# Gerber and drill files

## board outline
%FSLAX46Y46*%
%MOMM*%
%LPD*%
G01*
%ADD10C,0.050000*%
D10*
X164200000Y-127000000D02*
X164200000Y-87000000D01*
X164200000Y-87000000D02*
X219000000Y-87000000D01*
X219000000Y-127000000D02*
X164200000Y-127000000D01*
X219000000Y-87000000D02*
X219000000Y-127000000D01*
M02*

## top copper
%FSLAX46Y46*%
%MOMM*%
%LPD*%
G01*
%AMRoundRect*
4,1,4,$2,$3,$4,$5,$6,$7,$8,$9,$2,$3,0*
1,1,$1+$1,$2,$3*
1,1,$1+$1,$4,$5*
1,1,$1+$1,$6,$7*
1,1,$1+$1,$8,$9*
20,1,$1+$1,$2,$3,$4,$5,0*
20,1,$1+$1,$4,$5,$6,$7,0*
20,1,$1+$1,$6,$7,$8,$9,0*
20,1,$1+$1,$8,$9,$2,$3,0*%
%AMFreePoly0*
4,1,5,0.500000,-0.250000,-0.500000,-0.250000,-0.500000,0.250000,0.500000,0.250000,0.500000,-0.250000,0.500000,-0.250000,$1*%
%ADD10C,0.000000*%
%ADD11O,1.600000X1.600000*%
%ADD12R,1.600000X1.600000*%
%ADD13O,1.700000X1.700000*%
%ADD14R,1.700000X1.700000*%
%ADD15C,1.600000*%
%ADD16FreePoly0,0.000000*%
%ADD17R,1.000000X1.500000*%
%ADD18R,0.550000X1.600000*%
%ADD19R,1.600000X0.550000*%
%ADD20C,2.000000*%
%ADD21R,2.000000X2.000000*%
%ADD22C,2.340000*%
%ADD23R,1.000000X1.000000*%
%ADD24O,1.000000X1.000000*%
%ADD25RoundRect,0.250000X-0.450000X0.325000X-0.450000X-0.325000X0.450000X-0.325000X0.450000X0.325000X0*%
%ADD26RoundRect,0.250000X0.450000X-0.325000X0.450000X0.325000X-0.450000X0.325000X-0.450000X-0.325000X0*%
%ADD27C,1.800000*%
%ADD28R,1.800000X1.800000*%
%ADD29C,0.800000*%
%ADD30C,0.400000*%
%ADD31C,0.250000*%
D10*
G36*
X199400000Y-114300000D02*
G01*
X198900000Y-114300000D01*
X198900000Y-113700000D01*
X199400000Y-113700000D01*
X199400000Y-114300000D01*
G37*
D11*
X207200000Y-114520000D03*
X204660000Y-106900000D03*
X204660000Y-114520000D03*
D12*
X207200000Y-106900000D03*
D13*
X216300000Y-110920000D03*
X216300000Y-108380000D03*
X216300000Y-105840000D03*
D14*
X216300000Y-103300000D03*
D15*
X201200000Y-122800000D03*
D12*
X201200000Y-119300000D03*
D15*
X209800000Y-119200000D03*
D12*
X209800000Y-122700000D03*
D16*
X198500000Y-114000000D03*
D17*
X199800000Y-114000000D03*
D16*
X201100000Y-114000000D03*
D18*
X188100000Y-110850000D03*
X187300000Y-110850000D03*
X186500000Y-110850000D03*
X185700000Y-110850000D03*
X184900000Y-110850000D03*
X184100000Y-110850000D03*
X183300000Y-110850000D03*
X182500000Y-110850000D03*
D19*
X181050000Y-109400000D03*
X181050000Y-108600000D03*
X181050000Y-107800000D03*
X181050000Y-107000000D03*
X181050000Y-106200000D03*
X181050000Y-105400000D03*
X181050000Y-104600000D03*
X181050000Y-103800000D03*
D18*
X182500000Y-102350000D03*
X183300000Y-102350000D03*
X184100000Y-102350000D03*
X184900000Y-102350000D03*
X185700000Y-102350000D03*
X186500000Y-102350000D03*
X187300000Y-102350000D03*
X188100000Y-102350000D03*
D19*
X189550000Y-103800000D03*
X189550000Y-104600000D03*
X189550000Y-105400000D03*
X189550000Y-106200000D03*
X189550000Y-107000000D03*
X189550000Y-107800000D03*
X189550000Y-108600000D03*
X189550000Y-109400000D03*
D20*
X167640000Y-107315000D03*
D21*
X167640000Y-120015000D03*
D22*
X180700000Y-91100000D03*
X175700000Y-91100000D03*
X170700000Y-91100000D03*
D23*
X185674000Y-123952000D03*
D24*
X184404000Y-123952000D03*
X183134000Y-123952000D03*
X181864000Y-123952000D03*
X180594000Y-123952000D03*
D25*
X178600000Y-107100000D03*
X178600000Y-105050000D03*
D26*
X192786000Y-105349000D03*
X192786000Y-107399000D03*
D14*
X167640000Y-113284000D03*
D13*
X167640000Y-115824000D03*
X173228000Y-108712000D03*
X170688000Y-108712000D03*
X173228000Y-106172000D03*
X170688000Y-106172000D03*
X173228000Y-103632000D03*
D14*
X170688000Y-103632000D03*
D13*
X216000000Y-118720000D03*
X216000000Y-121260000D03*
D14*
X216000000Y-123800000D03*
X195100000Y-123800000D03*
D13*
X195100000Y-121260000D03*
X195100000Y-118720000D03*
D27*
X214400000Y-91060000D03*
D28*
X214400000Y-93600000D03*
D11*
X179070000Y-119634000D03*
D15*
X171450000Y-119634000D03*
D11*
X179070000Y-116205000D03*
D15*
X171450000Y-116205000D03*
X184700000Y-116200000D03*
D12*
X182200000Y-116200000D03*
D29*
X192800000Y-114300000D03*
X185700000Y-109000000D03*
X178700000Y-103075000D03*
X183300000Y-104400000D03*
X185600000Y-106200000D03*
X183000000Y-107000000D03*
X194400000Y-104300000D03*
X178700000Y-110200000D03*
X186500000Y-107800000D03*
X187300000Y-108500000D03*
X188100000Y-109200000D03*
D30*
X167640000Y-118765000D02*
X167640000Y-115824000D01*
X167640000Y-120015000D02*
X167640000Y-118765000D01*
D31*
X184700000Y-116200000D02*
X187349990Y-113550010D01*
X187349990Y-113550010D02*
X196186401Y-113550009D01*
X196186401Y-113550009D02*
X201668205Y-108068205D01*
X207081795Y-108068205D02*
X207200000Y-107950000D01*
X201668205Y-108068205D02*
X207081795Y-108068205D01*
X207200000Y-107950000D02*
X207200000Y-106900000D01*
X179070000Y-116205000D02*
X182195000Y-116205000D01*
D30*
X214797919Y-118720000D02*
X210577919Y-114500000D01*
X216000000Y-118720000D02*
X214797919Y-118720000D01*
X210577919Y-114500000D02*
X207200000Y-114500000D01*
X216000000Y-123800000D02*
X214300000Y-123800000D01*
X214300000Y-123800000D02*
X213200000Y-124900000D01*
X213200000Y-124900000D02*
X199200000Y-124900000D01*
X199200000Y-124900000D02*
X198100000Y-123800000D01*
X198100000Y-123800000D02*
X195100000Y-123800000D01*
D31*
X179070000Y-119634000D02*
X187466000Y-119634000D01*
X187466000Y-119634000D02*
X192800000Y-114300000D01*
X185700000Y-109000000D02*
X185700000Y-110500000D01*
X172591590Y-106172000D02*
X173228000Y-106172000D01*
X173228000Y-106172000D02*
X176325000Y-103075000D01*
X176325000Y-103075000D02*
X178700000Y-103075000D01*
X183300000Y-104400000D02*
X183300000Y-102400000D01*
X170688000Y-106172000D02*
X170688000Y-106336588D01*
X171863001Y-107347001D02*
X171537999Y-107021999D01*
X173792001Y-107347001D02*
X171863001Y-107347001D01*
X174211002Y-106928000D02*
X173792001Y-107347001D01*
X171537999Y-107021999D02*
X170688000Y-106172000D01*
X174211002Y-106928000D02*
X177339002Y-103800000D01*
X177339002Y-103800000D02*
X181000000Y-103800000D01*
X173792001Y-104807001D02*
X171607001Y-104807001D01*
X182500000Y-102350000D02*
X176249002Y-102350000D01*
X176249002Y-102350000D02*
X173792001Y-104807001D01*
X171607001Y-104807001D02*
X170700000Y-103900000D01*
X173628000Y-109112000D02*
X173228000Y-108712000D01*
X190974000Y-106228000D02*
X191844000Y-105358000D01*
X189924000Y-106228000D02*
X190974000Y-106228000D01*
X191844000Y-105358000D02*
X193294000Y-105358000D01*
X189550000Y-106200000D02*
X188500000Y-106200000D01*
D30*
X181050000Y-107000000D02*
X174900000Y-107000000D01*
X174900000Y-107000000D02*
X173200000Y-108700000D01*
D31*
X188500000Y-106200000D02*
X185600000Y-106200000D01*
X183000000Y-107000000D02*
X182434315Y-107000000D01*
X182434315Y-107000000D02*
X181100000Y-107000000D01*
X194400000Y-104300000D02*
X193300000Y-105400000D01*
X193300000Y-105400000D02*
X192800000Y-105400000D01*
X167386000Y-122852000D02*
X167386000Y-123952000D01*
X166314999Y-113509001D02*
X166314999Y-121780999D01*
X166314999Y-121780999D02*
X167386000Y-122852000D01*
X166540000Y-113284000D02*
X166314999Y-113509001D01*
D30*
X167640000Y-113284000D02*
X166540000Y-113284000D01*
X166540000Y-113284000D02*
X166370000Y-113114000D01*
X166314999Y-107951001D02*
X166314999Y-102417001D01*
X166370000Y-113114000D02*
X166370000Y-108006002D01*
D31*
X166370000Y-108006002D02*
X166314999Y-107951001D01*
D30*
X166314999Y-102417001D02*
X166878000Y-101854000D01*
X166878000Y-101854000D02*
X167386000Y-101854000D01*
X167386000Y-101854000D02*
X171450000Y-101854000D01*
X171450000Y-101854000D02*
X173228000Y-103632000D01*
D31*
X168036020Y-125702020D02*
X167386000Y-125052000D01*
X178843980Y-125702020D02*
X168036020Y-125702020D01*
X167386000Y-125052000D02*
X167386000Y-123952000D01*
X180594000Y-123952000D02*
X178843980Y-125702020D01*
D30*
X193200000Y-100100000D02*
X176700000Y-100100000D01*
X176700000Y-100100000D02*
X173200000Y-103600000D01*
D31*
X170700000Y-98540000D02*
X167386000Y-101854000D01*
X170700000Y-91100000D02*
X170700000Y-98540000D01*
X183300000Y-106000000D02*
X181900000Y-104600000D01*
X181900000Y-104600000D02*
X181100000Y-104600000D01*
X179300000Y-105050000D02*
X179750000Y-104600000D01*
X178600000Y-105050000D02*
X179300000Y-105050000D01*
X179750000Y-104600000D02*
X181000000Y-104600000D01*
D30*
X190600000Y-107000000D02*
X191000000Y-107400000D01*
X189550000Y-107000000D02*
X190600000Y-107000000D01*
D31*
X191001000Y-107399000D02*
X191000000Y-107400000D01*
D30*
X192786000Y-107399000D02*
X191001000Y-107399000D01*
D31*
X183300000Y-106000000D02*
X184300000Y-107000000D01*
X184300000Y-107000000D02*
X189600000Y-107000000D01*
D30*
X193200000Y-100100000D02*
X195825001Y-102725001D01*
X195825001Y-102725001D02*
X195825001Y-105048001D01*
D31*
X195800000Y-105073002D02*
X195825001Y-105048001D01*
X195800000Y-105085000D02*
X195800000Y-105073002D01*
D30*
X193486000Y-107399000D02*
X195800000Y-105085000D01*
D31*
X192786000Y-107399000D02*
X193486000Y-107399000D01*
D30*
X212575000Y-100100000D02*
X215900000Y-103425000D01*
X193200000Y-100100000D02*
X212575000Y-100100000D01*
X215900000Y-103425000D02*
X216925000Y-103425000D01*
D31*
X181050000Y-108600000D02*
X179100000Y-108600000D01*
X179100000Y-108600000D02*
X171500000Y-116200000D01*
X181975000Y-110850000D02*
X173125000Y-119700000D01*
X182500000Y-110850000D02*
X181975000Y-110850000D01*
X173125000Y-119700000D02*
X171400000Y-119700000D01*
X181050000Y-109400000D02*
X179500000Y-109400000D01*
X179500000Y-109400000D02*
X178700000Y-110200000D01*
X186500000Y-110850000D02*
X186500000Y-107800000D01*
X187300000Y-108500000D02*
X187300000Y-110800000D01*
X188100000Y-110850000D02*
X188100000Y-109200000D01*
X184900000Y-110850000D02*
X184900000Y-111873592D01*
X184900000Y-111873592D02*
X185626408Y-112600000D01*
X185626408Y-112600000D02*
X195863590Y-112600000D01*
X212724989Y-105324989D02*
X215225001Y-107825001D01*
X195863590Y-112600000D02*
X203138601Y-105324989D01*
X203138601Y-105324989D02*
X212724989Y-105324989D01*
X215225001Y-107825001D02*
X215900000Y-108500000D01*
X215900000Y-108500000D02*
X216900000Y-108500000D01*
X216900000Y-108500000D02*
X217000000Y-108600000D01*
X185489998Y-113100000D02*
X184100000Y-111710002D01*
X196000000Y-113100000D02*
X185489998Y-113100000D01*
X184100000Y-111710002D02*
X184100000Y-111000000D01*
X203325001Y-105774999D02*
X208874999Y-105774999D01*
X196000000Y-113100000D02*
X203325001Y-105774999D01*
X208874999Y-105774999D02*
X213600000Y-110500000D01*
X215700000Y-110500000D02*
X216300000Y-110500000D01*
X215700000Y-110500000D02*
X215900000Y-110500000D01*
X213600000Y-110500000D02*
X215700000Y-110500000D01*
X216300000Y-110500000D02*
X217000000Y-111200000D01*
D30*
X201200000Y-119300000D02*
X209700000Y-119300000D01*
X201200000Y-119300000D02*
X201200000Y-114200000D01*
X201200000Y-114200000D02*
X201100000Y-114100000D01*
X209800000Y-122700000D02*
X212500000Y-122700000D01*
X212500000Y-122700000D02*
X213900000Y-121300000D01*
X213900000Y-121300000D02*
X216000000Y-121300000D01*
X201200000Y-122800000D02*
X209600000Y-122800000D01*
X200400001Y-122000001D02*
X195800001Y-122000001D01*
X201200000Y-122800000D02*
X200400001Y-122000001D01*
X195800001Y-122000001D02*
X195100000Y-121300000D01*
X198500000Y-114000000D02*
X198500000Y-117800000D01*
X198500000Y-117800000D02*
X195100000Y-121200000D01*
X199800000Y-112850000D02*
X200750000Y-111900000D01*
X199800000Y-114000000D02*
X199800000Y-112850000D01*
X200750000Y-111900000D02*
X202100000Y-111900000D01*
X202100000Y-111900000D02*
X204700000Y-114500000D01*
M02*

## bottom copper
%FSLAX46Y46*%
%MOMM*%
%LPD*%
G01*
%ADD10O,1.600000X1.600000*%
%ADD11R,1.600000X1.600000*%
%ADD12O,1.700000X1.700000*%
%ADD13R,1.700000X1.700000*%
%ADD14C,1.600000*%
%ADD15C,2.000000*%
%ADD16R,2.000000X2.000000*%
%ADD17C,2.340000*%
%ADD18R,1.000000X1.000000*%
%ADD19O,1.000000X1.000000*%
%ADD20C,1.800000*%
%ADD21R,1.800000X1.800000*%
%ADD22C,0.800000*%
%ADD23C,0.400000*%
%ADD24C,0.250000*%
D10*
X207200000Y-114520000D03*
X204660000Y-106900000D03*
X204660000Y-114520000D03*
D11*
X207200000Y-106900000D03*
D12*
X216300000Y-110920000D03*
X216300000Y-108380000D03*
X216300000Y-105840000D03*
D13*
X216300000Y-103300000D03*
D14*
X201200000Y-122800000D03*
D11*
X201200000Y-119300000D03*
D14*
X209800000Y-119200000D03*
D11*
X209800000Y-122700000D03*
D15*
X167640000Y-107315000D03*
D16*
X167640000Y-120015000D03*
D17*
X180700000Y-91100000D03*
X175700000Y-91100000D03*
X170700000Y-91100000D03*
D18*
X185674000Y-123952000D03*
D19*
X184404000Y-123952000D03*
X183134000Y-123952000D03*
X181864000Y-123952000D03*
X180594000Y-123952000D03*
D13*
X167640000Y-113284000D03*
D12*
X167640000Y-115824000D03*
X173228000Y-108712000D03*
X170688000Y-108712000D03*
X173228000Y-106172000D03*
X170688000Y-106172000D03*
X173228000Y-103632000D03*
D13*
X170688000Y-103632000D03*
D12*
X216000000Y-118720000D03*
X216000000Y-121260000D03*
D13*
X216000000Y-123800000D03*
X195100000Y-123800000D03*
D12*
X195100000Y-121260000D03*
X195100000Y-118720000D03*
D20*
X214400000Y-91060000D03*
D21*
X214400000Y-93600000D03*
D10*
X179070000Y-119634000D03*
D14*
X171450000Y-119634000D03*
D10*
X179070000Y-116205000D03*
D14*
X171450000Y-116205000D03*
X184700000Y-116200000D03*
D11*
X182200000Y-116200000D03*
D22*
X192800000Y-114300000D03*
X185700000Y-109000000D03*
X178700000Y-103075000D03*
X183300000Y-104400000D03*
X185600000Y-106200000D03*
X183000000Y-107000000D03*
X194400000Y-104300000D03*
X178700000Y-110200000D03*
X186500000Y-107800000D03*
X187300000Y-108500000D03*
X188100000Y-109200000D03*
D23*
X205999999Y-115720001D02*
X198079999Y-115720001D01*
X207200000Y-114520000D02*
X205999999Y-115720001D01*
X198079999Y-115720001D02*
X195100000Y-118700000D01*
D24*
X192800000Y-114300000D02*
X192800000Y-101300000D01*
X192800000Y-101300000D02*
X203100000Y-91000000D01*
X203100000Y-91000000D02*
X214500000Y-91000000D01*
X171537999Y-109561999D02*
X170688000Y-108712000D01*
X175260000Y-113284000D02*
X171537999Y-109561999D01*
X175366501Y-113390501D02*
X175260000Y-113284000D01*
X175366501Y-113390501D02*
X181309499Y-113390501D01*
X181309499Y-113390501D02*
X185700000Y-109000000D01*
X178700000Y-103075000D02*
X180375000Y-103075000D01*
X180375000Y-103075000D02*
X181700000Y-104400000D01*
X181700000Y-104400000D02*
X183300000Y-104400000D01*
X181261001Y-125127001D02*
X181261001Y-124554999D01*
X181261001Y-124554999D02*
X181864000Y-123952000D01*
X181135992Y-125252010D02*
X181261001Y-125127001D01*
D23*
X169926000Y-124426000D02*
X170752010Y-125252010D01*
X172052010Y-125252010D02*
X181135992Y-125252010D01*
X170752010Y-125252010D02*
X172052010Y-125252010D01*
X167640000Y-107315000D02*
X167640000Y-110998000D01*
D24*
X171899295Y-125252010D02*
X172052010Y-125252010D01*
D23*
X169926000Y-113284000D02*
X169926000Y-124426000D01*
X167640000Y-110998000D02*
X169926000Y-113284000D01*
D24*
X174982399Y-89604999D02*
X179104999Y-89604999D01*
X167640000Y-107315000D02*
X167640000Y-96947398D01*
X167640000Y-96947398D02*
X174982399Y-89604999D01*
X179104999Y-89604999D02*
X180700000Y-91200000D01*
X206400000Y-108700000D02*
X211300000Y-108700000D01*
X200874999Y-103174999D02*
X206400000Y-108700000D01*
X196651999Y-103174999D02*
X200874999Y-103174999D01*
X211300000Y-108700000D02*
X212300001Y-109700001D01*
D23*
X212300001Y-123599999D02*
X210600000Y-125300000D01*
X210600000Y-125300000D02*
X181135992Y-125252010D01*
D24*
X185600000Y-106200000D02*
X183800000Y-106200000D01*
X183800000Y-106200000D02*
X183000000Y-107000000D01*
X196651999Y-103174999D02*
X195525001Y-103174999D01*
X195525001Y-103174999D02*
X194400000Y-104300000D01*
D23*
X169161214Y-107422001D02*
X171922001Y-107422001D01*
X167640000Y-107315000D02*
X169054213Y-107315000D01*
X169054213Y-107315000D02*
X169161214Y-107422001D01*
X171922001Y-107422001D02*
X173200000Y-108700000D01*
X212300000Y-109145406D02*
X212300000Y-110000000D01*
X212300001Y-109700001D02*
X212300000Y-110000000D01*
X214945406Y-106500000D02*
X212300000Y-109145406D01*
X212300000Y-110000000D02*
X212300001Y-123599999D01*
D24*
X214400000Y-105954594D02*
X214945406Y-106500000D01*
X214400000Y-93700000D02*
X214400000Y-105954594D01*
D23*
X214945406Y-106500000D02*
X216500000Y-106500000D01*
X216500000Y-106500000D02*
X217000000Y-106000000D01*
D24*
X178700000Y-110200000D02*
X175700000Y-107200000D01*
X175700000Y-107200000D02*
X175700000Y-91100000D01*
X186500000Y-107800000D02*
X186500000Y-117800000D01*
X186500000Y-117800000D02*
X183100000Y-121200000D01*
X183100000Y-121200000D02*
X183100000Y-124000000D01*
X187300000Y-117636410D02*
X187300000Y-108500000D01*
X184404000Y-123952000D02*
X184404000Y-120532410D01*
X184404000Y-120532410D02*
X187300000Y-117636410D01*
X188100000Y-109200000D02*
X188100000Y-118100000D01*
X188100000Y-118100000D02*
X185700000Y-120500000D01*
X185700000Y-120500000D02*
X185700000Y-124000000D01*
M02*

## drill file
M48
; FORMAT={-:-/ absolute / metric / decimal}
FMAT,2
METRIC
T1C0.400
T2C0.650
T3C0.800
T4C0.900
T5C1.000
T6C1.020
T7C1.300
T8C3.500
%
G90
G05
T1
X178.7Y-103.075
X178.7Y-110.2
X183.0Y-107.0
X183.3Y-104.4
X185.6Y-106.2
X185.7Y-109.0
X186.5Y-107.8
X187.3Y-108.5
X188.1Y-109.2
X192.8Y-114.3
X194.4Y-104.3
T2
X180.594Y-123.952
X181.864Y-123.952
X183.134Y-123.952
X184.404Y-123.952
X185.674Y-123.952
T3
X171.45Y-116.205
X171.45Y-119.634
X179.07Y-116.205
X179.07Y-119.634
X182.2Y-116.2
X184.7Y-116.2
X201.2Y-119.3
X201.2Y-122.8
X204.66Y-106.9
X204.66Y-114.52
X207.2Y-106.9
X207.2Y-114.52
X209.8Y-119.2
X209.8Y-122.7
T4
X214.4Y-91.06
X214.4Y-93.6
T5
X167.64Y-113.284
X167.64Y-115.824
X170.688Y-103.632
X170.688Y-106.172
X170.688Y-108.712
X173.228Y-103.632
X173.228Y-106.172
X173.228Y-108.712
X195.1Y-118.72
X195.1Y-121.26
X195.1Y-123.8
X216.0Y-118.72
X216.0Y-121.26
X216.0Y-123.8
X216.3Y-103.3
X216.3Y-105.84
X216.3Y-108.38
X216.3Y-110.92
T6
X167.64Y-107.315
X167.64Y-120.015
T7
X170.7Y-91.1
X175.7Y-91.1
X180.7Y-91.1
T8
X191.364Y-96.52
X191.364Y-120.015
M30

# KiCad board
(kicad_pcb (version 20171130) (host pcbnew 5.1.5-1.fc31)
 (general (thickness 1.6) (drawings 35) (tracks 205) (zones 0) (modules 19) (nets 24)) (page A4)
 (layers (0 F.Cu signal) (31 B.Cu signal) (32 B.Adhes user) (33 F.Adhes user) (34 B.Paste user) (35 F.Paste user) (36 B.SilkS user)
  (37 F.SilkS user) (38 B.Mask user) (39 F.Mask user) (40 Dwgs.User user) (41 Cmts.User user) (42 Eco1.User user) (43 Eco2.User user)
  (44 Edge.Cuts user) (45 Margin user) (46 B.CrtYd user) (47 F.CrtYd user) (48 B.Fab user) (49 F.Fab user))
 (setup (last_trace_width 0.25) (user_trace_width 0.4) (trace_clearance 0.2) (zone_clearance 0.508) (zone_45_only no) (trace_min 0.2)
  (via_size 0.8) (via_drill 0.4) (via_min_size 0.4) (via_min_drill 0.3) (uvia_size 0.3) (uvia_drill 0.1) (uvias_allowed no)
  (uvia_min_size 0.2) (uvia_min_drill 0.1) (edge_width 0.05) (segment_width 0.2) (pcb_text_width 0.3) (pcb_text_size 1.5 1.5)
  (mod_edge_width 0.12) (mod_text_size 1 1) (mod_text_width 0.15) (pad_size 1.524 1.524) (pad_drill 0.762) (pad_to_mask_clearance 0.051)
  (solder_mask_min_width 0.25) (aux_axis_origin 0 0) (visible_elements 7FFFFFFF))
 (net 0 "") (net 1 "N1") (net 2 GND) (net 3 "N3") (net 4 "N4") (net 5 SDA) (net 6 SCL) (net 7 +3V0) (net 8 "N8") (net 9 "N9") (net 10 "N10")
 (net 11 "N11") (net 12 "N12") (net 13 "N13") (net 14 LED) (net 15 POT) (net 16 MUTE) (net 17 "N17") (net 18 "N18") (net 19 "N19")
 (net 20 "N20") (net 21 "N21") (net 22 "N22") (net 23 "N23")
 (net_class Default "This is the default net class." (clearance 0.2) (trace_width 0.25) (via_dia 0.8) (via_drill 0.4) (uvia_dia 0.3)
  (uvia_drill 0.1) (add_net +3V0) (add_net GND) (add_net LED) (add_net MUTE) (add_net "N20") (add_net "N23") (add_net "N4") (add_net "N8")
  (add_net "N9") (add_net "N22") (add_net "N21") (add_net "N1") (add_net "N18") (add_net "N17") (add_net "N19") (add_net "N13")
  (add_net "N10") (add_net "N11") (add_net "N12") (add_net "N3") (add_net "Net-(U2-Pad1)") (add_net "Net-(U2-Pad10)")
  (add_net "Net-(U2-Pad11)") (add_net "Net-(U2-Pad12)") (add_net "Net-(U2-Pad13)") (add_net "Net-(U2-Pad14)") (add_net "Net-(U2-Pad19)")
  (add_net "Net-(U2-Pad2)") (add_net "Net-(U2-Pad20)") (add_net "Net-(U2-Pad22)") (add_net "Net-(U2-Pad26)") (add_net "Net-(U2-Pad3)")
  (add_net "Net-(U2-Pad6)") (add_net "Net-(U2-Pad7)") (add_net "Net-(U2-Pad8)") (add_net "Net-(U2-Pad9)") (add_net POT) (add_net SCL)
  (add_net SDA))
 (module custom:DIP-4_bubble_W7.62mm (layer F.Cu) (at 207.2 106.9 270)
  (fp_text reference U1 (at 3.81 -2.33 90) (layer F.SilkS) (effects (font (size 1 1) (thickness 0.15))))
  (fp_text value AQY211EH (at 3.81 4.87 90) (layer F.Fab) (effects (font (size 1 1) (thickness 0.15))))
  (pad 4 thru_hole oval (at 7.62 0 270) (size 1.6 1.6) (drill 0.8) (layers *.Cu *.Mask) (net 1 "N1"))
  (pad 2 thru_hole oval (at 0 2.54 270) (size 1.6 1.6) (drill 0.8) (layers *.Cu *.Mask) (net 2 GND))
  (pad 3 thru_hole oval (at 7.62 2.54 270) (size 1.6 1.6) (drill 0.8) (layers *.Cu *.Mask) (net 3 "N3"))
  (pad 1 thru_hole rect (at 0 0 270) (size 1.6 1.6) (drill 0.8) (layers *.Cu *.Mask) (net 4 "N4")))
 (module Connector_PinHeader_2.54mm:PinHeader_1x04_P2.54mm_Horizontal (layer F.Cu) (at 216.3 103.3)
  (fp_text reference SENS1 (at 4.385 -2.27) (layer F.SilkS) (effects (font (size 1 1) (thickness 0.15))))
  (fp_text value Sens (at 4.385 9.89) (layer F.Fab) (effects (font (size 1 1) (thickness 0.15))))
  (pad 4 thru_hole oval (at 0 7.62) (size 1.7 1.7) (drill 1) (layers *.Cu *.Mask) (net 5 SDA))
  (pad 3 thru_hole oval (at 0 5.08) (size 1.7 1.7) (drill 1) (layers *.Cu *.Mask) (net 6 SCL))
  (pad 2 thru_hole oval (at 0 2.54) (size 1.7 1.7) (drill 1) (layers *.Cu *.Mask) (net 2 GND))
  (pad 1 thru_hole rect (at 0 0) (size 1.7 1.7) (drill 1) (layers *.Cu *.Mask) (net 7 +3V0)))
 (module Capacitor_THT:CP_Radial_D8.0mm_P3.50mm (layer F.Cu) (at 201.2 119.3 270)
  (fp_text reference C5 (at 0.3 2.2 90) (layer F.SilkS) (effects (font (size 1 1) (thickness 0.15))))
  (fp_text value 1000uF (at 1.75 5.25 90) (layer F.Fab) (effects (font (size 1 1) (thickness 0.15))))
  (pad 2 thru_hole circle (at 3.5 0 270) (size 1.6 1.6) (drill 0.8) (layers *.Cu *.Mask) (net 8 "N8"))
  (pad 1 thru_hole rect (at 0 0 270) (size 1.6 1.6) (drill 0.8) (layers *.Cu *.Mask) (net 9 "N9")))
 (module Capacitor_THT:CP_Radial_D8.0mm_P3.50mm (layer F.Cu) (at 209.8 122.7 90)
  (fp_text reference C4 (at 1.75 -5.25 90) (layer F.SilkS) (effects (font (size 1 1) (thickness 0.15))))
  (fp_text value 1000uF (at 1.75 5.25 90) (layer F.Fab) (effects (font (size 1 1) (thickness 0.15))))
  (pad 2 thru_hole circle (at 3.5 0 90) (size 1.6 1.6) (drill 0.8) (layers *.Cu *.Mask) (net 9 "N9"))
  (pad 1 thru_hole rect (at 0 0 90) (size 1.6 1.6) (drill 0.8) (layers *.Cu *.Mask) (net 8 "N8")))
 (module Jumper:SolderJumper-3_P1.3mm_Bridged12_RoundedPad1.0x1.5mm (layer F.Cu) (at 199.8 114)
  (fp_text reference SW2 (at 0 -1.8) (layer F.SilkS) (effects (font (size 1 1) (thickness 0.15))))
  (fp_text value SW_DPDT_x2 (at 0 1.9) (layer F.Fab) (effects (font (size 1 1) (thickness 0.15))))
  (fp_poly (pts (xy -0.9 -0.3) (xy -0.4 -0.3) (xy -0.4 0.3) (xy -0.9 0.3)) (layer F.Cu) (width 0))
  (pad 1 smd custom (at -1.3 0) (size 1 0.5) (layers F.Cu F.Mask) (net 8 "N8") (zone_connect 2) (options (clearance outline) (anchor rect))
   (primitives))
  (pad 2 smd rect (at 0 0) (size 1 1.5) (layers F.Cu F.Mask) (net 3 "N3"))
  (pad 3 smd custom (at 1.3 0) (size 1 0.5) (layers F.Cu F.Mask) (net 9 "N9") (zone_connect 2) (options (clearance outline) (anchor rect))
   (primitives)))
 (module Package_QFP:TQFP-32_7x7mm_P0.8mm (layer F.Cu) (at 185.3 106.6 180)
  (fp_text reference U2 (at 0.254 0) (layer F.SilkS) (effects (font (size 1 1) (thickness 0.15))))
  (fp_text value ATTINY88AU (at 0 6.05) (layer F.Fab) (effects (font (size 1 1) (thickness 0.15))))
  (pad 32 smd rect (at -2.8 -4.25 270) (size 1.6 0.55) (layers F.Cu F.Paste F.Mask) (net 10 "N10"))
  (pad 31 smd rect (at -2 -4.25 270) (size 1.6 0.55) (layers F.Cu F.Paste F.Mask) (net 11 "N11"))
  (pad 30 smd rect (at -1.2 -4.25 270) (size 1.6 0.55) (layers F.Cu F.Paste F.Mask) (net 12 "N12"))
  (pad 29 smd rect (at -0.4 -4.25 270) (size 1.6 0.55) (layers F.Cu F.Paste F.Mask) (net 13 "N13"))
  (pad 28 smd rect (at 0.4 -4.25 270) (size 1.6 0.55) (layers F.Cu F.Paste F.Mask) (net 6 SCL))
  (pad 27 smd rect (at 1.2 -4.25 270) (size 1.6 0.55) (layers F.Cu F.Paste F.Mask) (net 5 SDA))
  (pad 26 smd rect (at 2 -4.25 270) (size 1.6 0.55) (layers F.Cu F.Paste F.Mask))
  (pad 25 smd rect (at 2.8 -4.25 270) (size 1.6 0.55) (layers F.Cu F.Paste F.Mask) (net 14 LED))
  (pad 24 smd rect (at 4.25 -2.8 180) (size 1.6 0.55) (layers F.Cu F.Paste F.Mask) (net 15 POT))
  (pad 23 smd rect (at 4.25 -2 180) (size 1.6 0.55) (layers F.Cu F.Paste F.Mask) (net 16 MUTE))
  (pad 22 smd rect (at 4.25 -1.2 180) (size 1.6 0.55) (layers F.Cu F.Paste F.Mask))
  (pad 21 smd rect (at 4.25 -0.4 180) (size 1.6 0.55) (layers F.Cu F.Paste F.Mask) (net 2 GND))
  (pad 20 smd rect (at 4.25 0.4 180) (size 1.6 0.55) (layers F.Cu F.Paste F.Mask))
  (pad 19 smd rect (at 4.25 1.2 180) (size 1.6 0.55) (layers F.Cu F.Paste F.Mask))
  (pad 18 smd rect (at 4.25 2 180) (size 1.6 0.55) (layers F.Cu F.Paste F.Mask) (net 7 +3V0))
  (pad 17 smd rect (at 4.25 2.8 180) (size 1.6 0.55) (layers F.Cu F.Paste F.Mask) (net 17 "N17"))
  (pad 16 smd rect (at 2.8 4.25 270) (size 1.6 0.55) (layers F.Cu F.Paste F.Mask) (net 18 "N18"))
  (pad 15 smd rect (at 2 4.25 270) (size 1.6 0.55) (layers F.Cu F.Paste F.Mask) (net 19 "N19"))
  (pad 14 smd rect (at 1.2 4.25 270) (size 1.6 0.55) (layers F.Cu F.Paste F.Mask))
  (pad 13 smd rect (at 0.4 4.25 270) (size 1.6 0.55) (layers F.Cu F.Paste F.Mask))
  (pad 12 smd rect (at -0.4 4.25 270) (size 1.6 0.55) (layers F.Cu F.Paste F.Mask))
  (pad 11 smd rect (at -1.2 4.25 270) (size 1.6 0.55) (layers F.Cu F.Paste F.Mask))
  (pad 10 smd rect (at -2 4.25 270) (size 1.6 0.55) (layers F.Cu F.Paste F.Mask))
  (pad 9 smd rect (at -2.8 4.25 270) (size 1.6 0.55) (layers F.Cu F.Paste F.Mask))
  (pad 8 smd rect (at -4.25 2.8 180) (size 1.6 0.55) (layers F.Cu F.Paste F.Mask))
  (pad 7 smd rect (at -4.25 2 180) (size 1.6 0.55) (layers F.Cu F.Paste F.Mask))
  (pad 6 smd rect (at -4.25 1.2 180) (size 1.6 0.55) (layers F.Cu F.Paste F.Mask))
  (pad 5 smd rect (at -4.25 0.4 180) (size 1.6 0.55) (layers F.Cu F.Paste F.Mask) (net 2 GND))
  (pad 4 smd rect (at -4.25 -0.4 180) (size 1.6 0.55) (layers F.Cu F.Paste F.Mask) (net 7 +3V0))
  (pad 3 smd rect (at -4.25 -1.2 180) (size 1.6 0.55) (layers F.Cu F.Paste F.Mask))
  (pad 2 smd rect (at -4.25 -2 180) (size 1.6 0.55) (layers F.Cu F.Paste F.Mask))
  (pad 1 smd rect (at -4.25 -2.8 180) (size 1.6 0.55) (layers F.Cu F.Paste F.Mask)))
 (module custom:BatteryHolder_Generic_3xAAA (layer B.Cu) (at 167.64 120.015)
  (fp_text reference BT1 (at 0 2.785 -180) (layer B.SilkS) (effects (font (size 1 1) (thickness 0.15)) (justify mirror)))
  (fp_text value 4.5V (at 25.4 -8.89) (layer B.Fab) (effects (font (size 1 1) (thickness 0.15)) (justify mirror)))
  (pad "" np_thru_hole circle (at 23.7236 0) (size 3.5 3.5) (drill 3.5) (layers *.Cu *.Mask))
  (pad "" np_thru_hole circle (at 23.7236 -23.495) (size 3.5 3.5) (drill 3.5) (layers *.Cu *.Mask))
  (pad 2 thru_hole circle (at 0 -12.7) (size 2 2) (drill 1.02) (layers *.Cu *.Mask) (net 2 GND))
  (pad 1 thru_hole rect (at 0 0) (size 2 2) (drill 1.02) (layers *.Cu *.Mask) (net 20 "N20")))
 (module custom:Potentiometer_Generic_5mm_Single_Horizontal (layer F.Cu) (at 180.7 91.1 90)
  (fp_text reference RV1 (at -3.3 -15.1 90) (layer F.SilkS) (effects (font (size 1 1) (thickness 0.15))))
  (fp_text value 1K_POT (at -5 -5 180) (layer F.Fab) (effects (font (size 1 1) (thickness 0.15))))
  (pad 1 thru_hole circle (at 0 0 90) (size 2.34 2.34) (drill 1.3) (layers *.Cu *.Mask) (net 2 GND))
  (pad 2 thru_hole circle (at 0 -5 90) (size 2.34 2.34) (drill 1.3) (layers *.Cu *.Mask) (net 15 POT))
  (pad 3 thru_hole circle (at 0 -10 90) (size 2.34 2.34) (drill 1.3) (layers *.Cu *.Mask) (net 7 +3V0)))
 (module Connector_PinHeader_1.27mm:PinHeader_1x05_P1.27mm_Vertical (layer F.Cu) (at 185.674 123.952 270)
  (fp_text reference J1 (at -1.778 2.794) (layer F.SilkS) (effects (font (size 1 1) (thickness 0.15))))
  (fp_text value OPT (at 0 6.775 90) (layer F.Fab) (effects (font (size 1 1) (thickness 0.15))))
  (pad 1 thru_hole rect (at 0 0 270) (size 1 1) (drill 0.65) (layers *.Cu *.Mask) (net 10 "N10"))
  (pad 2 thru_hole oval (at 0 1.27 270) (size 1 1) (drill 0.65) (layers *.Cu *.Mask) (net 11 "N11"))
  (pad 3 thru_hole oval (at 0 2.54 270) (size 1 1) (drill 0.65) (layers *.Cu *.Mask) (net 12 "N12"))
  (pad 4 thru_hole oval (at 0 3.81 270) (size 1 1) (drill 0.65) (layers *.Cu *.Mask) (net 2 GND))
  (pad 5 thru_hole oval (at 0 5.08 270) (size 1 1) (drill 0.65) (layers *.Cu *.Mask) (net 7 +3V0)))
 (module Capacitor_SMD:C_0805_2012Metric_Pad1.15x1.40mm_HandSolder (layer F.Cu) (at 178.6 106.075 270)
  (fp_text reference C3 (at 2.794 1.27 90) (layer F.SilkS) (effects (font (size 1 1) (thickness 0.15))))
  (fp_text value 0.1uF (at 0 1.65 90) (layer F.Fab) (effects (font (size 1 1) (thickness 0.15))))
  (pad 2 smd roundrect (at 1.025 0 270) (size 1.15 1.4) (layers F.Cu F.Paste F.Mask) (roundrect_rratio 0.217391) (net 2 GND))
  (pad 1 smd roundrect (at -1.025 0 270) (size 1.15 1.4) (layers F.Cu F.Paste F.Mask) (roundrect_rratio 0.217391) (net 7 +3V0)))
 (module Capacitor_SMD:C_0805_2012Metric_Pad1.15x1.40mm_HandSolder (layer F.Cu) (at 192.786 106.374 90)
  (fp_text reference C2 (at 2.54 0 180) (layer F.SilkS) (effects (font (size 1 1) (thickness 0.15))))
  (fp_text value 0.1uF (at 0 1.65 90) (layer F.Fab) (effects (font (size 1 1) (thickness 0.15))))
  (pad 2 smd roundrect (at 1.025 0 90) (size 1.15 1.4) (layers F.Cu F.Paste F.Mask) (roundrect_rratio 0.217391) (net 2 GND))
  (pad 1 smd roundrect (at -1.025 0 90) (size 1.15 1.4) (layers F.Cu F.Paste F.Mask) (roundrect_rratio 0.217391) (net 7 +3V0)))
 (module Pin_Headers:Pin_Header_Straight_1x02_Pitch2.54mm (layer F.Cu) (at 167.64 113.284)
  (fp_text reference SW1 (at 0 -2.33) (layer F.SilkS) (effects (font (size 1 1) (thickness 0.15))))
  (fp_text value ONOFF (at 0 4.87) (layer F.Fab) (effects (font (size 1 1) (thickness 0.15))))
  (pad 1 thru_hole rect (at 0 0) (size 1.7 1.7) (drill 1) (layers *.Cu *.Mask) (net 7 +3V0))
  (pad 2 thru_hole oval (at 0 2.54) (size 1.7 1.7) (drill 1) (layers *.Cu *.Mask) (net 20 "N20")))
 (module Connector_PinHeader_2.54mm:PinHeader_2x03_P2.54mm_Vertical (layer F.Cu) (at 170.688 103.632)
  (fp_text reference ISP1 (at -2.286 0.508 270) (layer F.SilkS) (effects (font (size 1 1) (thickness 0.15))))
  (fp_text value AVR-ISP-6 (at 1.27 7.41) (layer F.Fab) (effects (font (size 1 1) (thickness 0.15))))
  (pad 6 thru_hole oval (at 2.54 5.08) (size 1.7 1.7) (drill 1) (layers *.Cu *.Mask) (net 2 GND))
  (pad 5 thru_hole oval (at 0 5.08) (size 1.7 1.7) (drill 1) (layers *.Cu *.Mask) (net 13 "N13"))
  (pad 4 thru_hole oval (at 2.54 2.54) (size 1.7 1.7) (drill 1) (layers *.Cu *.Mask) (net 19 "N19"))
  (pad 3 thru_hole oval (at 0 2.54) (size 1.7 1.7) (drill 1) (layers *.Cu *.Mask) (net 17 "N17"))
  (pad 2 thru_hole oval (at 2.54 0) (size 1.7 1.7) (drill 1) (layers *.Cu *.Mask) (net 7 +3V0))
  (pad 1 thru_hole rect (at 0 0) (size 1.7 1.7) (drill 1) (layers *.Cu *.Mask) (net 18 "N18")))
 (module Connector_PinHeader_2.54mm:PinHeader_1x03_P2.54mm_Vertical (layer F.Cu) (at 216 123.8 180)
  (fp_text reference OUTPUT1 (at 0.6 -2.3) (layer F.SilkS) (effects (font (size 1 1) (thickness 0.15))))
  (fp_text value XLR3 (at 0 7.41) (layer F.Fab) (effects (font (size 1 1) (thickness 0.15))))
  (pad 3 thru_hole oval (at 0 5.08 180) (size 1.7 1.7) (drill 1) (layers *.Cu *.Mask) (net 1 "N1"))
  (pad 2 thru_hole oval (at 0 2.54 180) (size 1.7 1.7) (drill 1) (layers *.Cu *.Mask) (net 8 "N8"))
  (pad 1 thru_hole rect (at 0 0 180) (size 1.7 1.7) (drill 1) (layers *.Cu *.Mask) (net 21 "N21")))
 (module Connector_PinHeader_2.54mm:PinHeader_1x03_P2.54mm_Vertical (layer F.Cu) (at 195.1 123.8 180)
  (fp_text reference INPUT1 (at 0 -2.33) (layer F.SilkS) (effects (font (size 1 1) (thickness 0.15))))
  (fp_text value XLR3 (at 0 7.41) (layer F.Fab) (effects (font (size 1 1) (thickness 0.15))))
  (pad 1 thru_hole rect (at 0 0 180) (size 1.7 1.7) (drill 1) (layers *.Cu *.Mask) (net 21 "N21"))
  (pad 2 thru_hole oval (at 0 2.54 180) (size 1.7 1.7) (drill 1) (layers *.Cu *.Mask) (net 8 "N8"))
  (pad 3 thru_hole oval (at 0 5.08 180) (size 1.7 1.7) (drill 1) (layers *.Cu *.Mask) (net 1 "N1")))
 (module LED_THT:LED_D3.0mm (layer F.Cu) (at 214.4 93.6 90)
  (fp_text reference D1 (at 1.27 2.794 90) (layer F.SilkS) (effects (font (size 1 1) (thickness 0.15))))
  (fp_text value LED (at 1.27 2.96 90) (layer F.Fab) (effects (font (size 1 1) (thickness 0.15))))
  (pad 2 thru_hole circle (at 2.54 0 90) (size 1.8 1.8) (drill 0.9) (layers *.Cu *.Mask) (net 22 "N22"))
  (pad 1 thru_hole rect (at 0 0 90) (size 1.8 1.8) (drill 0.9) (layers *.Cu *.Mask) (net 2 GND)))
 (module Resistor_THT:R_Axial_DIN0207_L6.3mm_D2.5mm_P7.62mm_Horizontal (layer F.Cu) (at 171.45 119.634)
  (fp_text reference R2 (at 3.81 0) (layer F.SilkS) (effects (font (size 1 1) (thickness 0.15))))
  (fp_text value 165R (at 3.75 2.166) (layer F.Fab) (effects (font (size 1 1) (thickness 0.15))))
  (pad 2 thru_hole oval (at 7.62 0) (size 1.6 1.6) (drill 0.8) (layers *.Cu *.Mask) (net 22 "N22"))
  (pad 1 thru_hole circle (at 0 0) (size 1.6 1.6) (drill 0.8) (layers *.Cu *.Mask) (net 14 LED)))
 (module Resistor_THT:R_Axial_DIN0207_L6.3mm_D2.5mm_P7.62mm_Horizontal (layer F.Cu) (at 171.45 116.205)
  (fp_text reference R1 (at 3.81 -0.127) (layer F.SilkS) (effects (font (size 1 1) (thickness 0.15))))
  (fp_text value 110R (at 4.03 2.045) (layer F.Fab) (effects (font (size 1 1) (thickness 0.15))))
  (pad 2 thru_hole oval (at 7.62 0) (size 1.6 1.6) (drill 0.8) (layers *.Cu *.Mask) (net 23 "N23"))
  (pad 1 thru_hole circle (at 0 0) (size 1.6 1.6) (drill 0.8) (layers *.Cu *.Mask) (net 16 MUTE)))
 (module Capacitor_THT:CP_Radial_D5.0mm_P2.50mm (layer F.Cu) (at 182.2 116.2)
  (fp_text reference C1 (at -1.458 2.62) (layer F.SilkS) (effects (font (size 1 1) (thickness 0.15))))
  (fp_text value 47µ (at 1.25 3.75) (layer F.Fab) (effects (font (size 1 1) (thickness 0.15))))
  (pad 2 thru_hole circle (at 2.5 0) (size 1.6 1.6) (drill 0.8) (layers *.Cu *.Mask) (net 4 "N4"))
  (pad 1 thru_hole rect (at 0 0) (size 1.6 1.6) (drill 0.8) (layers *.Cu *.Mask) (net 23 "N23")))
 (gr_line (start 164.2 127) (end 164.2 87) (layer Edge.Cuts) (width 0.05))
 (gr_line (start 164.2 87) (end 219 87) (layer Edge.Cuts) (width 0.05))
 (gr_line (start 219 127) (end 164.2 127) (layer Edge.Cuts) (width 0.05))
 (gr_line (start 219 87) (end 219 127) (layer Edge.Cuts) (width 0.05))
 (segment (start 167.64 118.765) (end 167.64 115.824) (width 0.4) (layer F.Cu) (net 20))
 (segment (start 167.64 120.015) (end 167.64 118.765) (width 0.4) (layer F.Cu) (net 20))
 (segment (start 184.7 116.2) (end 187.34999 113.55001) (width 0.25) (layer F.Cu) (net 4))
 (segment (start 187.34999 113.55001) (end 196.186401 113.550009) (width 0.25) (layer F.Cu) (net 4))
 (segment (start 196.186401 113.550009) (end 201.668205 108.068205) (width 0.25) (layer F.Cu) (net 4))
 (segment (start 207.081795 108.068205) (end 207.2 107.95) (width 0.25) (layer F.Cu) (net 4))
 (segment (start 201.668205 108.068205) (end 207.081795 108.068205) (width 0.25) (layer F.Cu) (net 4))
 (segment (start 207.2 107.95) (end 207.2 106.9) (width 0.25) (layer F.Cu) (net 4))
 (segment (start 179.07 116.205) (end 182.195 116.205) (width 0.25) (layer F.Cu) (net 23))
 (segment (start 214.797919 118.72) (end 210.577919 114.5) (width 0.4) (layer F.Cu) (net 1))
 (segment (start 216 118.72) (end 214.797919 118.72) (width 0.4) (layer F.Cu) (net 1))
 (segment (start 210.577919 114.5) (end 207.2 114.5) (width 0.4) (layer F.Cu) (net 1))
 (segment (start 205.999999 115.720001) (end 198.079999 115.720001) (width 0.4) (layer B.Cu) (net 1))
 (segment (start 207.2 114.52) (end 205.999999 115.720001) (width 0.4) (layer B.Cu) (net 1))
 (segment (start 198.079999 115.720001) (end 195.1 118.7) (width 0.4) (layer B.Cu) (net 1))
 (segment (start 216 123.8) (end 214.3 123.8) (width 0.4) (layer F.Cu) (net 21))
 (segment (start 214.3 123.8) (end 213.2 124.9) (width 0.4) (layer F.Cu) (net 21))
 (segment (start 213.2 124.9) (end 199.2 124.9) (width 0.4) (layer F.Cu) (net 21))
 (segment (start 199.2 124.9) (end 198.1 123.8) (width 0.4) (layer F.Cu) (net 21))
 (segment (start 198.1 123.8) (end 195.1 123.8) (width 0.4) (layer F.Cu) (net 21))
 (via (at 192.8 114.3) (size 0.8) (drill 0.4) (layers F.Cu B.Cu) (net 22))
 (segment (start 179.07 119.634) (end 187.466 119.634) (width 0.25) (layer F.Cu) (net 22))
 (segment (start 187.466 119.634) (end 192.8 114.3) (width 0.25) (layer F.Cu) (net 22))
 (segment (start 192.8 114.3) (end 192.8 101.3) (width 0.25) (layer B.Cu) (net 22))
 (segment (start 192.8 101.3) (end 203.1 91) (width 0.25) (layer B.Cu) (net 22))
 (segment (start 203.1 91) (end 214.5 91) (width 0.25) (layer B.Cu) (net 22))
 (segment (start 171.537999 109.561999) (end 170.688 108.712) (width 0.25) (layer B.Cu) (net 13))
 (segment (start 175.26 113.284) (end 171.537999 109.561999) (width 0.25) (layer B.Cu) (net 13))
 (segment (start 175.366501 113.390501) (end 175.26 113.284) (width 0.25) (layer B.Cu) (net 13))
 (via (at 185.7 109) (size 0.8) (drill 0.4) (layers F.Cu B.Cu) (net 13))
 (segment (start 175.366501 113.390501) (end 181.309499 113.390501) (width 0.25) (layer B.Cu) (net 13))
 (segment (start 181.309499 113.390501) (end 185.7 109) (width 0.25) (layer B.Cu) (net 13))
 (segment (start 185.7 109) (end 185.7 110.5) (width 0.25) (layer F.Cu) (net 13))
 (segment (start 172.59159 106.172) (end 173.228 106.172) (width 0.25) (layer F.Cu) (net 19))
 (via (at 178.7 103.075) (size 0.8) (drill 0.4) (layers F.Cu B.Cu) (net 19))
 (segment (start 173.228 106.172) (end 176.325 103.075) (width 0.25) (layer F.Cu) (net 19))
 (segment (start 176.325 103.075) (end 178.7 103.075) (width 0.25) (layer F.Cu) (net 19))
 (segment (start 178.7 103.075) (end 180.375 103.075) (width 0.25) (layer B.Cu) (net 19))
 (via (at 183.3 104.4) (size 0.8) (drill 0.4) (layers F.Cu B.Cu) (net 19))
 (segment (start 180.375 103.075) (end 181.7 104.4) (width 0.25) (layer B.Cu) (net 19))
 (segment (start 181.7 104.4) (end 183.3 104.4) (width 0.25) (layer B.Cu) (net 19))
 (segment (start 183.3 104.4) (end 183.3 102.4) (width 0.25) (layer F.Cu) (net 19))
 (segment (start 170.688 106.172) (end 170.688 106.336588) (width 0.25) (layer F.Cu) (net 17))
 (segment (start 171.863001 107.347001) (end 171.537999 107.021999) (width 0.25) (layer F.Cu) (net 17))
 (segment (start 173.792001 107.347001) (end 171.863001 107.347001) (width 0.25) (layer F.Cu) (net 17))
 (segment (start 174.211002 106.928) (end 173.792001 107.347001) (width 0.25) (layer F.Cu) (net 17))
 (segment (start 171.537999 107.021999) (end 170.688 106.172) (width 0.25) (layer F.Cu) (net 17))
 (segment (start 174.211002 106.928) (end 177.339002 103.8) (width 0.25) (layer F.Cu) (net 17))
 (segment (start 177.339002 103.8) (end 181 103.8) (width 0.25) (layer F.Cu) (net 17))
 (segment (start 173.792001 104.807001) (end 171.607001 104.807001) (width 0.25) (layer F.Cu) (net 18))
 (segment (start 182.5 102.35) (end 176.249002 102.35) (width 0.25) (layer F.Cu) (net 18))
 (segment (start 176.249002 102.35) (end 173.792001 104.807001) (width 0.25) (layer F.Cu) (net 18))
 (segment (start 171.607001 104.807001) (end 170.7 103.9) (width 0.25) (layer F.Cu) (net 18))
 (segment (start 173.628 109.112) (end 173.228 108.712) (width 0.25) (layer F.Cu) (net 2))
 (segment (start 190.974 106.228) (end 191.844 105.358) (width 0.25) (layer F.Cu) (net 2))
 (segment (start 189.924 106.228) (end 190.974 106.228) (width 0.25) (layer F.Cu) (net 2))
 (segment (start 191.844 105.358) (end 193.294 105.358) (width 0.25) (layer F.Cu) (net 2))
 (segment (start 181.261001 125.127001) (end 181.261001 124.554999) (width 0.25) (layer B.Cu) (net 2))
 (segment (start 181.261001 124.554999) (end 181.864 123.952) (width 0.25) (layer B.Cu) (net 2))
 (segment (start 181.135992 125.25201) (end 181.261001 125.127001) (width 0.25) (layer B.Cu) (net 2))
 (segment (start 189.55 106.2) (end 188.5 106.2) (width 0.25) (layer F.Cu) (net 2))
 (segment (start 181.05 107) (end 174.9 107) (width 0.4) (layer F.Cu) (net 2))
 (segment (start 174.9 107) (end 173.2 108.7) (width 0.4) (layer F.Cu) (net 2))
 (segment (start 169.926 124.426) (end 170.75201 125.25201) (width 0.4) (layer B.Cu) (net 2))
 (segment (start 172.05201 125.25201) (end 181.135992 125.25201) (width 0.4) (layer B.Cu) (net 2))
 (segment (start 170.75201 125.25201) (end 172.05201 125.25201) (width 0.4) (layer B.Cu) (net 2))
 (segment (start 167.64 107.315) (end 167.64 110.998) (width 0.4) (layer B.Cu) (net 2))
 (segment (start 171.899295 125.25201) (end 172.05201 125.25201) (width 0.25) (layer B.Cu) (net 2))
 (segment (start 169.926 113.284) (end 169.926 124.426) (width 0.4) (layer B.Cu) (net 2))
 (segment (start 167.64 110.998) (end 169.926 113.284) (width 0.4) (layer B.Cu) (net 2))
 (segment (start 174.982399 89.604999) (end 179.104999 89.604999) (width 0.25) (layer B.Cu) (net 2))
 (segment (start 167.64 107.315) (end 167.64 96.947398) (width 0.25) (layer B.Cu) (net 2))
 (segment (start 167.64 96.947398) (end 174.982399 89.604999) (width 0.25) (layer B.Cu) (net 2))
 (segment (start 179.104999 89.604999) (end 180.7 91.2) (width 0.25) (layer B.Cu) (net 2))
 (segment (start 206.4 108.7) (end 211.3 108.7) (width 0.25) (layer B.Cu) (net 2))
 (segment (start 200.874999 103.174999) (end 206.4 108.7) (width 0.25) (layer B.Cu) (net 2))
 (segment (start 196.651999 103.174999) (end 200.874999 103.174999) (width 0.25) (layer B.Cu) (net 2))
 (segment (start 211.3 108.7) (end 212.300001 109.700001) (width 0.25) (layer B.Cu) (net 2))
 (segment (start 212.300001 123.599999) (end 210.6 125.3) (width 0.4) (layer B.Cu) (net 2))
 (segment (start 210.6 125.3) (end 181.135992 125.25201) (width 0.4) (layer B.Cu) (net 2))
 (via (at 185.6 106.2) (size 0.8) (drill 0.4) (layers F.Cu B.Cu) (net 2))
 (segment (start 188.5 106.2) (end 185.6 106.2) (width 0.25) (layer F.Cu) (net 2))
 (via (at 183 107) (size 0.8) (drill 0.4) (layers F.Cu B.Cu) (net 2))
 (segment (start 185.6 106.2) (end 183.8 106.2) (width 0.25) (layer B.Cu) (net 2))
 (segment (start 183.8 106.2) (end 183 107) (width 0.25) (layer B.Cu) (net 2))
 (segment (start 183 107) (end 182.434315 107) (width 0.25) (layer F.Cu) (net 2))
 (segment (start 182.434315 107) (end 181.1 107) (width 0.25) (layer F.Cu) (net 2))
 (segment (start 196.651999 103.174999) (end 195.525001 103.174999) (width 0.25) (layer B.Cu) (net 2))
 (via (at 194.4 104.3) (size 0.8) (drill 0.4) (layers F.Cu B.Cu) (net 2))
 (segment (start 195.525001 103.174999) (end 194.4 104.3) (width 0.25) (layer B.Cu) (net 2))
 (segment (start 194.4 104.3) (end 193.3 105.4) (width 0.25) (layer F.Cu) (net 2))
 (segment (start 193.3 105.4) (end 192.8 105.4) (width 0.25) (layer F.Cu) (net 2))
 (segment (start 169.161214 107.422001) (end 171.922001 107.422001) (width 0.4) (layer B.Cu) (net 2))
 (segment (start 167.64 107.315) (end 169.054213 107.315) (width 0.4) (layer B.Cu) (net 2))
 (segment (start 169.054213 107.315) (end 169.161214 107.422001) (width 0.4) (layer B.Cu) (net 2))
 (segment (start 171.922001 107.422001) (end 173.2 108.7) (width 0.4) (layer B.Cu) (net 2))
 (segment (start 212.3 109.145406) (end 212.3 110) (width 0.4) (layer B.Cu) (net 2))
 (segment (start 212.300001 109.700001) (end 212.3 110) (width 0.4) (layer B.Cu) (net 2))
 (segment (start 214.945406 106.5) (end 212.3 109.145406) (width 0.4) (layer B.Cu) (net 2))
 (segment (start 212.3 110) (end 212.300001 123.599999) (width 0.4) (layer B.Cu) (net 2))
 (segment (start 214.4 105.954594) (end 214.945406 106.5) (width 0.25) (layer B.Cu) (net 2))
 (segment (start 214.4 93.7) (end 214.4 105.954594) (width 0.25) (layer B.Cu) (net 2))
 (segment (start 214.945406 106.5) (end 216.5 106.5) (width 0.4) (layer B.Cu) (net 2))
 (segment (start 216.5 106.5) (end 217 106) (width 0.4) (layer B.Cu) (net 2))
 (segment (start 167.386 122.852) (end 167.386 123.952) (width 0.25) (layer F.Cu) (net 7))
 (segment (start 166.314999 113.509001) (end 166.314999 121.780999) (width 0.25) (layer F.Cu) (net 7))
 (segment (start 166.314999 121.780999) (end 167.386 122.852) (width 0.25) (layer F.Cu) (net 7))
 (segment (start 166.54 113.284) (end 166.314999 113.509001) (width 0.25) (layer F.Cu) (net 7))
 (segment (start 167.64 113.284) (end 166.54 113.284) (width 0.4) (layer F.Cu) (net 7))
 (segment (start 166.54 113.284) (end 166.37 113.114) (width 0.4) (layer F.Cu) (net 7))
 (segment (start 166.314999 107.951001) (end 166.314999 102.417001) (width 0.4) (layer F.Cu) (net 7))
 (segment (start 166.37 113.114) (end 166.37 108.006002) (width 0.4) (layer F.Cu) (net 7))
 (segment (start 166.37 108.006002) (end 166.314999 107.951001) (width 0.25) (layer F.Cu) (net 7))
 (segment (start 166.314999 102.417001) (end 166.878 101.854) (width 0.4) (layer F.Cu) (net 7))
 (segment (start 166.878 101.854) (end 167.386 101.854) (width 0.4) (layer F.Cu) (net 7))
 (segment (start 167.386 101.854) (end 171.45 101.854) (width 0.4) (layer F.Cu) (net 7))
 (segment (start 171.45 101.854) (end 173.228 103.632) (width 0.4) (layer F.Cu) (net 7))
 (segment (start 168.03602 125.70202) (end 167.386 125.052) (width 0.25) (layer F.Cu) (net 7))
 (segment (start 178.84398 125.70202) (end 168.03602 125.70202) (width 0.25) (layer F.Cu) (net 7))
 (segment (start 167.386 125.052) (end 167.386 123.952) (width 0.25) (layer F.Cu) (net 7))
 (segment (start 180.594 123.952) (end 178.84398 125.70202) (width 0.25) (layer F.Cu) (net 7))
 (segment (start 193.2 100.1) (end 176.7 100.1) (width 0.4) (layer F.Cu) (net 7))
 (segment (start 176.7 100.1) (end 173.2 103.6) (width 0.4) (layer F.Cu) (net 7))
 (segment (start 170.7 98.54) (end 167.386 101.854) (width 0.25) (layer F.Cu) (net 7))
 (segment (start 170.7 91.1) (end 170.7 98.54) (width 0.25) (layer F.Cu) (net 7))
 (segment (start 183.3 106) (end 181.9 104.6) (width 0.25) (layer F.Cu) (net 7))
 (segment (start 181.9 104.6) (end 181.1 104.6) (width 0.25) (layer F.Cu) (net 7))
 (segment (start 179.3 105.05) (end 179.75 104.6) (width 0.25) (layer F.Cu) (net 7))
 (segment (start 178.6 105.05) (end 179.3 105.05) (width 0.25) (layer F.Cu) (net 7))
 (segment (start 179.75 104.6) (end 181 104.6) (width 0.25) (layer F.Cu) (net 7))
 (segment (start 190.6 107) (end 191 107.4) (width 0.4) (layer F.Cu) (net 7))
 (segment (start 189.55 107) (end 190.6 107) (width 0.4) (layer F.Cu) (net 7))
 (segment (start 191.001 107.399) (end 191 107.4) (width 0.25) (layer F.Cu) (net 7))
 (segment (start 192.786 107.399) (end 191.001 107.399) (width 0.4) (layer F.Cu) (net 7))
 (segment (start 183.3 106) (end 184.3 107) (width 0.25) (layer F.Cu) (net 7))
 (segment (start 184.3 107) (end 189.6 107) (width 0.25) (layer F.Cu) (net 7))
 (segment (start 193.2 100.1) (end 195.825001 102.725001) (width 0.4) (layer F.Cu) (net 7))
 (segment (start 195.825001 102.725001) (end 195.825001 105.048001) (width 0.4) (layer F.Cu) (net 7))
 (segment (start 195.8 105.073002) (end 195.825001 105.048001) (width 0.25) (layer F.Cu) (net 7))
 (segment (start 195.8 105.085) (end 195.8 105.073002) (width 0.25) (layer F.Cu) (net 7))
 (segment (start 193.486 107.399) (end 195.8 105.085) (width 0.4) (layer F.Cu) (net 7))
 (segment (start 192.786 107.399) (end 193.486 107.399) (width 0.25) (layer F.Cu) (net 7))
 (segment (start 212.575 100.1) (end 215.9 103.425) (width 0.4) (layer F.Cu) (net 7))
 (segment (start 193.2 100.1) (end 212.575 100.1) (width 0.4) (layer F.Cu) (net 7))
 (segment (start 215.9 103.425) (end 216.925 103.425) (width 0.4) (layer F.Cu) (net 7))
 (segment (start 181.05 108.6) (end 179.1 108.6) (width 0.25) (layer F.Cu) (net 16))
 (segment (start 179.1 108.6) (end 171.5 116.2) (width 0.25) (layer F.Cu) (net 16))
 (segment (start 181.975 110.85) (end 173.125 119.7) (width 0.25) (layer F.Cu) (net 14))
 (segment (start 182.5 110.85) (end 181.975 110.85) (width 0.25) (layer F.Cu) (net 14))
 (segment (start 173.125 119.7) (end 171.4 119.7) (width 0.25) (layer F.Cu) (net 14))
 (via (at 178.7 110.2) (size 0.8) (drill 0.4) (layers F.Cu B.Cu) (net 15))
 (segment (start 181.05 109.4) (end 179.5 109.4) (width 0.25) (layer F.Cu) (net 15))
 (segment (start 179.5 109.4) (end 178.7 110.2) (width 0.25) (layer F.Cu) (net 15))
 (segment (start 178.7 110.2) (end 175.7 107.2) (width 0.25) (layer B.Cu) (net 15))
 (segment (start 175.7 107.2) (end 175.7 91.1) (width 0.25) (layer B.Cu) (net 15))
 (via (at 186.5 107.8) (size 0.8) (drill 0.4) (layers F.Cu B.Cu) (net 12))
 (segment (start 186.5 110.85) (end 186.5 107.8) (width 0.25) (layer F.Cu) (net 12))
 (segment (start 186.5 107.8) (end 186.5 117.8) (width 0.25) (layer B.Cu) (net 12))
 (segment (start 186.5 117.8) (end 183.1 121.2) (width 0.25) (layer B.Cu) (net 12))
 (segment (start 183.1 121.2) (end 183.1 124) (width 0.25) (layer B.Cu) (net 12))
 (segment (start 187.3 117.63641) (end 187.3 108.5) (width 0.25) (layer B.Cu) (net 11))
 (segment (start 184.404 123.952) (end 184.404 120.53241) (width 0.25) (layer B.Cu) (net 11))
 (via (at 187.3 108.5) (size 0.8) (drill 0.4) (layers F.Cu B.Cu) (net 11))
 (segment (start 184.404 120.53241) (end 187.3 117.63641) (width 0.25) (layer B.Cu) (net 11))
 (segment (start 187.3 108.5) (end 187.3 110.8) (width 0.25) (layer F.Cu) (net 11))
 (via (at 188.1 109.2) (size 0.8) (drill 0.4) (layers F.Cu B.Cu) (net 10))
 (segment (start 188.1 110.85) (end 188.1 109.2) (width 0.25) (layer F.Cu) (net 10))
 (segment (start 188.1 109.2) (end 188.1 118.1) (width 0.25) (layer B.Cu) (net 10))
 (segment (start 188.1 118.1) (end 185.7 120.5) (width 0.25) (layer B.Cu) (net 10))
 (segment (start 185.7 120.5) (end 185.7 124) (width 0.25) (layer B.Cu) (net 10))
 (segment (start 184.9 110.85) (end 184.9 111.873592) (width 0.25) (layer F.Cu) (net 6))
 (segment (start 184.9 111.873592) (end 185.626408 112.6) (width 0.25) (layer F.Cu) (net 6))
 (segment (start 185.626408 112.6) (end 195.86359 112.6) (width 0.25) (layer F.Cu) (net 6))
 (segment (start 212.724989 105.324989) (end 215.225001 107.825001) (width 0.25) (layer F.Cu) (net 6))
 (segment (start 195.86359 112.6) (end 203.138601 105.324989) (width 0.25) (layer F.Cu) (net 6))
 (segment (start 203.138601 105.324989) (end 212.724989 105.324989) (width 0.25) (layer F.Cu) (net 6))
 (segment (start 215.225001 107.825001) (end 215.9 108.5) (width 0.25) (layer F.Cu) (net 6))
 (segment (start 215.9 108.5) (end 216.9 108.5) (width 0.25) (layer F.Cu) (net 6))
 (segment (start 216.9 108.5) (end 217 108.6) (width 0.25) (layer F.Cu) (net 6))
 (segment (start 185.489998 113.1) (end 184.1 111.710002) (width 0.25) (layer F.Cu) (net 5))
 (segment (start 196 113.1) (end 185.489998 113.1) (width 0.25) (layer F.Cu) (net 5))
 (segment (start 184.1 111.710002) (end 184.1 111) (width 0.25) (layer F.Cu) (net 5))
 (segment (start 203.325001 105.774999) (end 208.874999 105.774999) (width 0.25) (layer F.Cu) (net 5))
 (segment (start 196 113.1) (end 203.325001 105.774999) (width 0.25) (layer F.Cu) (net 5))
 (segment (start 208.874999 105.774999) (end 213.6 110.5) (width 0.25) (layer F.Cu) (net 5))
 (segment (start 215.7 110.5) (end 216.3 110.5) (width 0.25) (layer F.Cu) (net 5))
 (segment (start 215.7 110.5) (end 215.9 110.5) (width 0.25) (layer F.Cu) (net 5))
 (segment (start 213.6 110.5) (end 215.7 110.5) (width 0.25) (layer F.Cu) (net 5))
 (segment (start 216.3 110.5) (end 217 111.2) (width 0.25) (layer F.Cu) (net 5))
 (segment (start 201.2 119.3) (end 209.7 119.3) (width 0.4) (layer F.Cu) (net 9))
 (segment (start 201.2 119.3) (end 201.2 114.2) (width 0.4) (layer F.Cu) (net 9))
 (segment (start 201.2 114.2) (end 201.1 114.1) (width 0.4) (layer F.Cu) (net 9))
 (segment (start 209.8 122.7) (end 212.5 122.7) (width 0.4) (layer F.Cu) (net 8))
 (segment (start 212.5 122.7) (end 213.9 121.3) (width 0.4) (layer F.Cu) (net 8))
 (segment (start 213.9 121.3) (end 216 121.3) (width 0.4) (layer F.Cu) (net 8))
 (segment (start 201.2 122.8) (end 209.6 122.8) (width 0.4) (layer F.Cu) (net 8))
 (segment (start 200.400001 122.000001) (end 195.800001 122.000001) (width 0.4) (layer F.Cu) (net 8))
 (segment (start 201.2 122.8) (end 200.400001 122.000001) (width 0.4) (layer F.Cu) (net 8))
 (segment (start 195.800001 122.000001) (end 195.1 121.3) (width 0.4) (layer F.Cu) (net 8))
 (segment (start 198.5 114) (end 198.5 117.8) (width 0.4) (layer F.Cu) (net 8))
 (segment (start 198.5 117.8) (end 195.1 121.2) (width 0.4) (layer F.Cu) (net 8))
 (segment (start 199.8 112.85) (end 200.75 111.9) (width 0.4) (layer F.Cu) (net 3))
 (segment (start 199.8 114) (end 199.8 112.85) (width 0.4) (layer F.Cu) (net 3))
 (segment (start 200.75 111.9) (end 202.1 111.9) (width 0.4) (layer F.Cu) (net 3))
 (segment (start 202.1 111.9) (end 204.7 114.5) (width 0.4) (layer F.Cu) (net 3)))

